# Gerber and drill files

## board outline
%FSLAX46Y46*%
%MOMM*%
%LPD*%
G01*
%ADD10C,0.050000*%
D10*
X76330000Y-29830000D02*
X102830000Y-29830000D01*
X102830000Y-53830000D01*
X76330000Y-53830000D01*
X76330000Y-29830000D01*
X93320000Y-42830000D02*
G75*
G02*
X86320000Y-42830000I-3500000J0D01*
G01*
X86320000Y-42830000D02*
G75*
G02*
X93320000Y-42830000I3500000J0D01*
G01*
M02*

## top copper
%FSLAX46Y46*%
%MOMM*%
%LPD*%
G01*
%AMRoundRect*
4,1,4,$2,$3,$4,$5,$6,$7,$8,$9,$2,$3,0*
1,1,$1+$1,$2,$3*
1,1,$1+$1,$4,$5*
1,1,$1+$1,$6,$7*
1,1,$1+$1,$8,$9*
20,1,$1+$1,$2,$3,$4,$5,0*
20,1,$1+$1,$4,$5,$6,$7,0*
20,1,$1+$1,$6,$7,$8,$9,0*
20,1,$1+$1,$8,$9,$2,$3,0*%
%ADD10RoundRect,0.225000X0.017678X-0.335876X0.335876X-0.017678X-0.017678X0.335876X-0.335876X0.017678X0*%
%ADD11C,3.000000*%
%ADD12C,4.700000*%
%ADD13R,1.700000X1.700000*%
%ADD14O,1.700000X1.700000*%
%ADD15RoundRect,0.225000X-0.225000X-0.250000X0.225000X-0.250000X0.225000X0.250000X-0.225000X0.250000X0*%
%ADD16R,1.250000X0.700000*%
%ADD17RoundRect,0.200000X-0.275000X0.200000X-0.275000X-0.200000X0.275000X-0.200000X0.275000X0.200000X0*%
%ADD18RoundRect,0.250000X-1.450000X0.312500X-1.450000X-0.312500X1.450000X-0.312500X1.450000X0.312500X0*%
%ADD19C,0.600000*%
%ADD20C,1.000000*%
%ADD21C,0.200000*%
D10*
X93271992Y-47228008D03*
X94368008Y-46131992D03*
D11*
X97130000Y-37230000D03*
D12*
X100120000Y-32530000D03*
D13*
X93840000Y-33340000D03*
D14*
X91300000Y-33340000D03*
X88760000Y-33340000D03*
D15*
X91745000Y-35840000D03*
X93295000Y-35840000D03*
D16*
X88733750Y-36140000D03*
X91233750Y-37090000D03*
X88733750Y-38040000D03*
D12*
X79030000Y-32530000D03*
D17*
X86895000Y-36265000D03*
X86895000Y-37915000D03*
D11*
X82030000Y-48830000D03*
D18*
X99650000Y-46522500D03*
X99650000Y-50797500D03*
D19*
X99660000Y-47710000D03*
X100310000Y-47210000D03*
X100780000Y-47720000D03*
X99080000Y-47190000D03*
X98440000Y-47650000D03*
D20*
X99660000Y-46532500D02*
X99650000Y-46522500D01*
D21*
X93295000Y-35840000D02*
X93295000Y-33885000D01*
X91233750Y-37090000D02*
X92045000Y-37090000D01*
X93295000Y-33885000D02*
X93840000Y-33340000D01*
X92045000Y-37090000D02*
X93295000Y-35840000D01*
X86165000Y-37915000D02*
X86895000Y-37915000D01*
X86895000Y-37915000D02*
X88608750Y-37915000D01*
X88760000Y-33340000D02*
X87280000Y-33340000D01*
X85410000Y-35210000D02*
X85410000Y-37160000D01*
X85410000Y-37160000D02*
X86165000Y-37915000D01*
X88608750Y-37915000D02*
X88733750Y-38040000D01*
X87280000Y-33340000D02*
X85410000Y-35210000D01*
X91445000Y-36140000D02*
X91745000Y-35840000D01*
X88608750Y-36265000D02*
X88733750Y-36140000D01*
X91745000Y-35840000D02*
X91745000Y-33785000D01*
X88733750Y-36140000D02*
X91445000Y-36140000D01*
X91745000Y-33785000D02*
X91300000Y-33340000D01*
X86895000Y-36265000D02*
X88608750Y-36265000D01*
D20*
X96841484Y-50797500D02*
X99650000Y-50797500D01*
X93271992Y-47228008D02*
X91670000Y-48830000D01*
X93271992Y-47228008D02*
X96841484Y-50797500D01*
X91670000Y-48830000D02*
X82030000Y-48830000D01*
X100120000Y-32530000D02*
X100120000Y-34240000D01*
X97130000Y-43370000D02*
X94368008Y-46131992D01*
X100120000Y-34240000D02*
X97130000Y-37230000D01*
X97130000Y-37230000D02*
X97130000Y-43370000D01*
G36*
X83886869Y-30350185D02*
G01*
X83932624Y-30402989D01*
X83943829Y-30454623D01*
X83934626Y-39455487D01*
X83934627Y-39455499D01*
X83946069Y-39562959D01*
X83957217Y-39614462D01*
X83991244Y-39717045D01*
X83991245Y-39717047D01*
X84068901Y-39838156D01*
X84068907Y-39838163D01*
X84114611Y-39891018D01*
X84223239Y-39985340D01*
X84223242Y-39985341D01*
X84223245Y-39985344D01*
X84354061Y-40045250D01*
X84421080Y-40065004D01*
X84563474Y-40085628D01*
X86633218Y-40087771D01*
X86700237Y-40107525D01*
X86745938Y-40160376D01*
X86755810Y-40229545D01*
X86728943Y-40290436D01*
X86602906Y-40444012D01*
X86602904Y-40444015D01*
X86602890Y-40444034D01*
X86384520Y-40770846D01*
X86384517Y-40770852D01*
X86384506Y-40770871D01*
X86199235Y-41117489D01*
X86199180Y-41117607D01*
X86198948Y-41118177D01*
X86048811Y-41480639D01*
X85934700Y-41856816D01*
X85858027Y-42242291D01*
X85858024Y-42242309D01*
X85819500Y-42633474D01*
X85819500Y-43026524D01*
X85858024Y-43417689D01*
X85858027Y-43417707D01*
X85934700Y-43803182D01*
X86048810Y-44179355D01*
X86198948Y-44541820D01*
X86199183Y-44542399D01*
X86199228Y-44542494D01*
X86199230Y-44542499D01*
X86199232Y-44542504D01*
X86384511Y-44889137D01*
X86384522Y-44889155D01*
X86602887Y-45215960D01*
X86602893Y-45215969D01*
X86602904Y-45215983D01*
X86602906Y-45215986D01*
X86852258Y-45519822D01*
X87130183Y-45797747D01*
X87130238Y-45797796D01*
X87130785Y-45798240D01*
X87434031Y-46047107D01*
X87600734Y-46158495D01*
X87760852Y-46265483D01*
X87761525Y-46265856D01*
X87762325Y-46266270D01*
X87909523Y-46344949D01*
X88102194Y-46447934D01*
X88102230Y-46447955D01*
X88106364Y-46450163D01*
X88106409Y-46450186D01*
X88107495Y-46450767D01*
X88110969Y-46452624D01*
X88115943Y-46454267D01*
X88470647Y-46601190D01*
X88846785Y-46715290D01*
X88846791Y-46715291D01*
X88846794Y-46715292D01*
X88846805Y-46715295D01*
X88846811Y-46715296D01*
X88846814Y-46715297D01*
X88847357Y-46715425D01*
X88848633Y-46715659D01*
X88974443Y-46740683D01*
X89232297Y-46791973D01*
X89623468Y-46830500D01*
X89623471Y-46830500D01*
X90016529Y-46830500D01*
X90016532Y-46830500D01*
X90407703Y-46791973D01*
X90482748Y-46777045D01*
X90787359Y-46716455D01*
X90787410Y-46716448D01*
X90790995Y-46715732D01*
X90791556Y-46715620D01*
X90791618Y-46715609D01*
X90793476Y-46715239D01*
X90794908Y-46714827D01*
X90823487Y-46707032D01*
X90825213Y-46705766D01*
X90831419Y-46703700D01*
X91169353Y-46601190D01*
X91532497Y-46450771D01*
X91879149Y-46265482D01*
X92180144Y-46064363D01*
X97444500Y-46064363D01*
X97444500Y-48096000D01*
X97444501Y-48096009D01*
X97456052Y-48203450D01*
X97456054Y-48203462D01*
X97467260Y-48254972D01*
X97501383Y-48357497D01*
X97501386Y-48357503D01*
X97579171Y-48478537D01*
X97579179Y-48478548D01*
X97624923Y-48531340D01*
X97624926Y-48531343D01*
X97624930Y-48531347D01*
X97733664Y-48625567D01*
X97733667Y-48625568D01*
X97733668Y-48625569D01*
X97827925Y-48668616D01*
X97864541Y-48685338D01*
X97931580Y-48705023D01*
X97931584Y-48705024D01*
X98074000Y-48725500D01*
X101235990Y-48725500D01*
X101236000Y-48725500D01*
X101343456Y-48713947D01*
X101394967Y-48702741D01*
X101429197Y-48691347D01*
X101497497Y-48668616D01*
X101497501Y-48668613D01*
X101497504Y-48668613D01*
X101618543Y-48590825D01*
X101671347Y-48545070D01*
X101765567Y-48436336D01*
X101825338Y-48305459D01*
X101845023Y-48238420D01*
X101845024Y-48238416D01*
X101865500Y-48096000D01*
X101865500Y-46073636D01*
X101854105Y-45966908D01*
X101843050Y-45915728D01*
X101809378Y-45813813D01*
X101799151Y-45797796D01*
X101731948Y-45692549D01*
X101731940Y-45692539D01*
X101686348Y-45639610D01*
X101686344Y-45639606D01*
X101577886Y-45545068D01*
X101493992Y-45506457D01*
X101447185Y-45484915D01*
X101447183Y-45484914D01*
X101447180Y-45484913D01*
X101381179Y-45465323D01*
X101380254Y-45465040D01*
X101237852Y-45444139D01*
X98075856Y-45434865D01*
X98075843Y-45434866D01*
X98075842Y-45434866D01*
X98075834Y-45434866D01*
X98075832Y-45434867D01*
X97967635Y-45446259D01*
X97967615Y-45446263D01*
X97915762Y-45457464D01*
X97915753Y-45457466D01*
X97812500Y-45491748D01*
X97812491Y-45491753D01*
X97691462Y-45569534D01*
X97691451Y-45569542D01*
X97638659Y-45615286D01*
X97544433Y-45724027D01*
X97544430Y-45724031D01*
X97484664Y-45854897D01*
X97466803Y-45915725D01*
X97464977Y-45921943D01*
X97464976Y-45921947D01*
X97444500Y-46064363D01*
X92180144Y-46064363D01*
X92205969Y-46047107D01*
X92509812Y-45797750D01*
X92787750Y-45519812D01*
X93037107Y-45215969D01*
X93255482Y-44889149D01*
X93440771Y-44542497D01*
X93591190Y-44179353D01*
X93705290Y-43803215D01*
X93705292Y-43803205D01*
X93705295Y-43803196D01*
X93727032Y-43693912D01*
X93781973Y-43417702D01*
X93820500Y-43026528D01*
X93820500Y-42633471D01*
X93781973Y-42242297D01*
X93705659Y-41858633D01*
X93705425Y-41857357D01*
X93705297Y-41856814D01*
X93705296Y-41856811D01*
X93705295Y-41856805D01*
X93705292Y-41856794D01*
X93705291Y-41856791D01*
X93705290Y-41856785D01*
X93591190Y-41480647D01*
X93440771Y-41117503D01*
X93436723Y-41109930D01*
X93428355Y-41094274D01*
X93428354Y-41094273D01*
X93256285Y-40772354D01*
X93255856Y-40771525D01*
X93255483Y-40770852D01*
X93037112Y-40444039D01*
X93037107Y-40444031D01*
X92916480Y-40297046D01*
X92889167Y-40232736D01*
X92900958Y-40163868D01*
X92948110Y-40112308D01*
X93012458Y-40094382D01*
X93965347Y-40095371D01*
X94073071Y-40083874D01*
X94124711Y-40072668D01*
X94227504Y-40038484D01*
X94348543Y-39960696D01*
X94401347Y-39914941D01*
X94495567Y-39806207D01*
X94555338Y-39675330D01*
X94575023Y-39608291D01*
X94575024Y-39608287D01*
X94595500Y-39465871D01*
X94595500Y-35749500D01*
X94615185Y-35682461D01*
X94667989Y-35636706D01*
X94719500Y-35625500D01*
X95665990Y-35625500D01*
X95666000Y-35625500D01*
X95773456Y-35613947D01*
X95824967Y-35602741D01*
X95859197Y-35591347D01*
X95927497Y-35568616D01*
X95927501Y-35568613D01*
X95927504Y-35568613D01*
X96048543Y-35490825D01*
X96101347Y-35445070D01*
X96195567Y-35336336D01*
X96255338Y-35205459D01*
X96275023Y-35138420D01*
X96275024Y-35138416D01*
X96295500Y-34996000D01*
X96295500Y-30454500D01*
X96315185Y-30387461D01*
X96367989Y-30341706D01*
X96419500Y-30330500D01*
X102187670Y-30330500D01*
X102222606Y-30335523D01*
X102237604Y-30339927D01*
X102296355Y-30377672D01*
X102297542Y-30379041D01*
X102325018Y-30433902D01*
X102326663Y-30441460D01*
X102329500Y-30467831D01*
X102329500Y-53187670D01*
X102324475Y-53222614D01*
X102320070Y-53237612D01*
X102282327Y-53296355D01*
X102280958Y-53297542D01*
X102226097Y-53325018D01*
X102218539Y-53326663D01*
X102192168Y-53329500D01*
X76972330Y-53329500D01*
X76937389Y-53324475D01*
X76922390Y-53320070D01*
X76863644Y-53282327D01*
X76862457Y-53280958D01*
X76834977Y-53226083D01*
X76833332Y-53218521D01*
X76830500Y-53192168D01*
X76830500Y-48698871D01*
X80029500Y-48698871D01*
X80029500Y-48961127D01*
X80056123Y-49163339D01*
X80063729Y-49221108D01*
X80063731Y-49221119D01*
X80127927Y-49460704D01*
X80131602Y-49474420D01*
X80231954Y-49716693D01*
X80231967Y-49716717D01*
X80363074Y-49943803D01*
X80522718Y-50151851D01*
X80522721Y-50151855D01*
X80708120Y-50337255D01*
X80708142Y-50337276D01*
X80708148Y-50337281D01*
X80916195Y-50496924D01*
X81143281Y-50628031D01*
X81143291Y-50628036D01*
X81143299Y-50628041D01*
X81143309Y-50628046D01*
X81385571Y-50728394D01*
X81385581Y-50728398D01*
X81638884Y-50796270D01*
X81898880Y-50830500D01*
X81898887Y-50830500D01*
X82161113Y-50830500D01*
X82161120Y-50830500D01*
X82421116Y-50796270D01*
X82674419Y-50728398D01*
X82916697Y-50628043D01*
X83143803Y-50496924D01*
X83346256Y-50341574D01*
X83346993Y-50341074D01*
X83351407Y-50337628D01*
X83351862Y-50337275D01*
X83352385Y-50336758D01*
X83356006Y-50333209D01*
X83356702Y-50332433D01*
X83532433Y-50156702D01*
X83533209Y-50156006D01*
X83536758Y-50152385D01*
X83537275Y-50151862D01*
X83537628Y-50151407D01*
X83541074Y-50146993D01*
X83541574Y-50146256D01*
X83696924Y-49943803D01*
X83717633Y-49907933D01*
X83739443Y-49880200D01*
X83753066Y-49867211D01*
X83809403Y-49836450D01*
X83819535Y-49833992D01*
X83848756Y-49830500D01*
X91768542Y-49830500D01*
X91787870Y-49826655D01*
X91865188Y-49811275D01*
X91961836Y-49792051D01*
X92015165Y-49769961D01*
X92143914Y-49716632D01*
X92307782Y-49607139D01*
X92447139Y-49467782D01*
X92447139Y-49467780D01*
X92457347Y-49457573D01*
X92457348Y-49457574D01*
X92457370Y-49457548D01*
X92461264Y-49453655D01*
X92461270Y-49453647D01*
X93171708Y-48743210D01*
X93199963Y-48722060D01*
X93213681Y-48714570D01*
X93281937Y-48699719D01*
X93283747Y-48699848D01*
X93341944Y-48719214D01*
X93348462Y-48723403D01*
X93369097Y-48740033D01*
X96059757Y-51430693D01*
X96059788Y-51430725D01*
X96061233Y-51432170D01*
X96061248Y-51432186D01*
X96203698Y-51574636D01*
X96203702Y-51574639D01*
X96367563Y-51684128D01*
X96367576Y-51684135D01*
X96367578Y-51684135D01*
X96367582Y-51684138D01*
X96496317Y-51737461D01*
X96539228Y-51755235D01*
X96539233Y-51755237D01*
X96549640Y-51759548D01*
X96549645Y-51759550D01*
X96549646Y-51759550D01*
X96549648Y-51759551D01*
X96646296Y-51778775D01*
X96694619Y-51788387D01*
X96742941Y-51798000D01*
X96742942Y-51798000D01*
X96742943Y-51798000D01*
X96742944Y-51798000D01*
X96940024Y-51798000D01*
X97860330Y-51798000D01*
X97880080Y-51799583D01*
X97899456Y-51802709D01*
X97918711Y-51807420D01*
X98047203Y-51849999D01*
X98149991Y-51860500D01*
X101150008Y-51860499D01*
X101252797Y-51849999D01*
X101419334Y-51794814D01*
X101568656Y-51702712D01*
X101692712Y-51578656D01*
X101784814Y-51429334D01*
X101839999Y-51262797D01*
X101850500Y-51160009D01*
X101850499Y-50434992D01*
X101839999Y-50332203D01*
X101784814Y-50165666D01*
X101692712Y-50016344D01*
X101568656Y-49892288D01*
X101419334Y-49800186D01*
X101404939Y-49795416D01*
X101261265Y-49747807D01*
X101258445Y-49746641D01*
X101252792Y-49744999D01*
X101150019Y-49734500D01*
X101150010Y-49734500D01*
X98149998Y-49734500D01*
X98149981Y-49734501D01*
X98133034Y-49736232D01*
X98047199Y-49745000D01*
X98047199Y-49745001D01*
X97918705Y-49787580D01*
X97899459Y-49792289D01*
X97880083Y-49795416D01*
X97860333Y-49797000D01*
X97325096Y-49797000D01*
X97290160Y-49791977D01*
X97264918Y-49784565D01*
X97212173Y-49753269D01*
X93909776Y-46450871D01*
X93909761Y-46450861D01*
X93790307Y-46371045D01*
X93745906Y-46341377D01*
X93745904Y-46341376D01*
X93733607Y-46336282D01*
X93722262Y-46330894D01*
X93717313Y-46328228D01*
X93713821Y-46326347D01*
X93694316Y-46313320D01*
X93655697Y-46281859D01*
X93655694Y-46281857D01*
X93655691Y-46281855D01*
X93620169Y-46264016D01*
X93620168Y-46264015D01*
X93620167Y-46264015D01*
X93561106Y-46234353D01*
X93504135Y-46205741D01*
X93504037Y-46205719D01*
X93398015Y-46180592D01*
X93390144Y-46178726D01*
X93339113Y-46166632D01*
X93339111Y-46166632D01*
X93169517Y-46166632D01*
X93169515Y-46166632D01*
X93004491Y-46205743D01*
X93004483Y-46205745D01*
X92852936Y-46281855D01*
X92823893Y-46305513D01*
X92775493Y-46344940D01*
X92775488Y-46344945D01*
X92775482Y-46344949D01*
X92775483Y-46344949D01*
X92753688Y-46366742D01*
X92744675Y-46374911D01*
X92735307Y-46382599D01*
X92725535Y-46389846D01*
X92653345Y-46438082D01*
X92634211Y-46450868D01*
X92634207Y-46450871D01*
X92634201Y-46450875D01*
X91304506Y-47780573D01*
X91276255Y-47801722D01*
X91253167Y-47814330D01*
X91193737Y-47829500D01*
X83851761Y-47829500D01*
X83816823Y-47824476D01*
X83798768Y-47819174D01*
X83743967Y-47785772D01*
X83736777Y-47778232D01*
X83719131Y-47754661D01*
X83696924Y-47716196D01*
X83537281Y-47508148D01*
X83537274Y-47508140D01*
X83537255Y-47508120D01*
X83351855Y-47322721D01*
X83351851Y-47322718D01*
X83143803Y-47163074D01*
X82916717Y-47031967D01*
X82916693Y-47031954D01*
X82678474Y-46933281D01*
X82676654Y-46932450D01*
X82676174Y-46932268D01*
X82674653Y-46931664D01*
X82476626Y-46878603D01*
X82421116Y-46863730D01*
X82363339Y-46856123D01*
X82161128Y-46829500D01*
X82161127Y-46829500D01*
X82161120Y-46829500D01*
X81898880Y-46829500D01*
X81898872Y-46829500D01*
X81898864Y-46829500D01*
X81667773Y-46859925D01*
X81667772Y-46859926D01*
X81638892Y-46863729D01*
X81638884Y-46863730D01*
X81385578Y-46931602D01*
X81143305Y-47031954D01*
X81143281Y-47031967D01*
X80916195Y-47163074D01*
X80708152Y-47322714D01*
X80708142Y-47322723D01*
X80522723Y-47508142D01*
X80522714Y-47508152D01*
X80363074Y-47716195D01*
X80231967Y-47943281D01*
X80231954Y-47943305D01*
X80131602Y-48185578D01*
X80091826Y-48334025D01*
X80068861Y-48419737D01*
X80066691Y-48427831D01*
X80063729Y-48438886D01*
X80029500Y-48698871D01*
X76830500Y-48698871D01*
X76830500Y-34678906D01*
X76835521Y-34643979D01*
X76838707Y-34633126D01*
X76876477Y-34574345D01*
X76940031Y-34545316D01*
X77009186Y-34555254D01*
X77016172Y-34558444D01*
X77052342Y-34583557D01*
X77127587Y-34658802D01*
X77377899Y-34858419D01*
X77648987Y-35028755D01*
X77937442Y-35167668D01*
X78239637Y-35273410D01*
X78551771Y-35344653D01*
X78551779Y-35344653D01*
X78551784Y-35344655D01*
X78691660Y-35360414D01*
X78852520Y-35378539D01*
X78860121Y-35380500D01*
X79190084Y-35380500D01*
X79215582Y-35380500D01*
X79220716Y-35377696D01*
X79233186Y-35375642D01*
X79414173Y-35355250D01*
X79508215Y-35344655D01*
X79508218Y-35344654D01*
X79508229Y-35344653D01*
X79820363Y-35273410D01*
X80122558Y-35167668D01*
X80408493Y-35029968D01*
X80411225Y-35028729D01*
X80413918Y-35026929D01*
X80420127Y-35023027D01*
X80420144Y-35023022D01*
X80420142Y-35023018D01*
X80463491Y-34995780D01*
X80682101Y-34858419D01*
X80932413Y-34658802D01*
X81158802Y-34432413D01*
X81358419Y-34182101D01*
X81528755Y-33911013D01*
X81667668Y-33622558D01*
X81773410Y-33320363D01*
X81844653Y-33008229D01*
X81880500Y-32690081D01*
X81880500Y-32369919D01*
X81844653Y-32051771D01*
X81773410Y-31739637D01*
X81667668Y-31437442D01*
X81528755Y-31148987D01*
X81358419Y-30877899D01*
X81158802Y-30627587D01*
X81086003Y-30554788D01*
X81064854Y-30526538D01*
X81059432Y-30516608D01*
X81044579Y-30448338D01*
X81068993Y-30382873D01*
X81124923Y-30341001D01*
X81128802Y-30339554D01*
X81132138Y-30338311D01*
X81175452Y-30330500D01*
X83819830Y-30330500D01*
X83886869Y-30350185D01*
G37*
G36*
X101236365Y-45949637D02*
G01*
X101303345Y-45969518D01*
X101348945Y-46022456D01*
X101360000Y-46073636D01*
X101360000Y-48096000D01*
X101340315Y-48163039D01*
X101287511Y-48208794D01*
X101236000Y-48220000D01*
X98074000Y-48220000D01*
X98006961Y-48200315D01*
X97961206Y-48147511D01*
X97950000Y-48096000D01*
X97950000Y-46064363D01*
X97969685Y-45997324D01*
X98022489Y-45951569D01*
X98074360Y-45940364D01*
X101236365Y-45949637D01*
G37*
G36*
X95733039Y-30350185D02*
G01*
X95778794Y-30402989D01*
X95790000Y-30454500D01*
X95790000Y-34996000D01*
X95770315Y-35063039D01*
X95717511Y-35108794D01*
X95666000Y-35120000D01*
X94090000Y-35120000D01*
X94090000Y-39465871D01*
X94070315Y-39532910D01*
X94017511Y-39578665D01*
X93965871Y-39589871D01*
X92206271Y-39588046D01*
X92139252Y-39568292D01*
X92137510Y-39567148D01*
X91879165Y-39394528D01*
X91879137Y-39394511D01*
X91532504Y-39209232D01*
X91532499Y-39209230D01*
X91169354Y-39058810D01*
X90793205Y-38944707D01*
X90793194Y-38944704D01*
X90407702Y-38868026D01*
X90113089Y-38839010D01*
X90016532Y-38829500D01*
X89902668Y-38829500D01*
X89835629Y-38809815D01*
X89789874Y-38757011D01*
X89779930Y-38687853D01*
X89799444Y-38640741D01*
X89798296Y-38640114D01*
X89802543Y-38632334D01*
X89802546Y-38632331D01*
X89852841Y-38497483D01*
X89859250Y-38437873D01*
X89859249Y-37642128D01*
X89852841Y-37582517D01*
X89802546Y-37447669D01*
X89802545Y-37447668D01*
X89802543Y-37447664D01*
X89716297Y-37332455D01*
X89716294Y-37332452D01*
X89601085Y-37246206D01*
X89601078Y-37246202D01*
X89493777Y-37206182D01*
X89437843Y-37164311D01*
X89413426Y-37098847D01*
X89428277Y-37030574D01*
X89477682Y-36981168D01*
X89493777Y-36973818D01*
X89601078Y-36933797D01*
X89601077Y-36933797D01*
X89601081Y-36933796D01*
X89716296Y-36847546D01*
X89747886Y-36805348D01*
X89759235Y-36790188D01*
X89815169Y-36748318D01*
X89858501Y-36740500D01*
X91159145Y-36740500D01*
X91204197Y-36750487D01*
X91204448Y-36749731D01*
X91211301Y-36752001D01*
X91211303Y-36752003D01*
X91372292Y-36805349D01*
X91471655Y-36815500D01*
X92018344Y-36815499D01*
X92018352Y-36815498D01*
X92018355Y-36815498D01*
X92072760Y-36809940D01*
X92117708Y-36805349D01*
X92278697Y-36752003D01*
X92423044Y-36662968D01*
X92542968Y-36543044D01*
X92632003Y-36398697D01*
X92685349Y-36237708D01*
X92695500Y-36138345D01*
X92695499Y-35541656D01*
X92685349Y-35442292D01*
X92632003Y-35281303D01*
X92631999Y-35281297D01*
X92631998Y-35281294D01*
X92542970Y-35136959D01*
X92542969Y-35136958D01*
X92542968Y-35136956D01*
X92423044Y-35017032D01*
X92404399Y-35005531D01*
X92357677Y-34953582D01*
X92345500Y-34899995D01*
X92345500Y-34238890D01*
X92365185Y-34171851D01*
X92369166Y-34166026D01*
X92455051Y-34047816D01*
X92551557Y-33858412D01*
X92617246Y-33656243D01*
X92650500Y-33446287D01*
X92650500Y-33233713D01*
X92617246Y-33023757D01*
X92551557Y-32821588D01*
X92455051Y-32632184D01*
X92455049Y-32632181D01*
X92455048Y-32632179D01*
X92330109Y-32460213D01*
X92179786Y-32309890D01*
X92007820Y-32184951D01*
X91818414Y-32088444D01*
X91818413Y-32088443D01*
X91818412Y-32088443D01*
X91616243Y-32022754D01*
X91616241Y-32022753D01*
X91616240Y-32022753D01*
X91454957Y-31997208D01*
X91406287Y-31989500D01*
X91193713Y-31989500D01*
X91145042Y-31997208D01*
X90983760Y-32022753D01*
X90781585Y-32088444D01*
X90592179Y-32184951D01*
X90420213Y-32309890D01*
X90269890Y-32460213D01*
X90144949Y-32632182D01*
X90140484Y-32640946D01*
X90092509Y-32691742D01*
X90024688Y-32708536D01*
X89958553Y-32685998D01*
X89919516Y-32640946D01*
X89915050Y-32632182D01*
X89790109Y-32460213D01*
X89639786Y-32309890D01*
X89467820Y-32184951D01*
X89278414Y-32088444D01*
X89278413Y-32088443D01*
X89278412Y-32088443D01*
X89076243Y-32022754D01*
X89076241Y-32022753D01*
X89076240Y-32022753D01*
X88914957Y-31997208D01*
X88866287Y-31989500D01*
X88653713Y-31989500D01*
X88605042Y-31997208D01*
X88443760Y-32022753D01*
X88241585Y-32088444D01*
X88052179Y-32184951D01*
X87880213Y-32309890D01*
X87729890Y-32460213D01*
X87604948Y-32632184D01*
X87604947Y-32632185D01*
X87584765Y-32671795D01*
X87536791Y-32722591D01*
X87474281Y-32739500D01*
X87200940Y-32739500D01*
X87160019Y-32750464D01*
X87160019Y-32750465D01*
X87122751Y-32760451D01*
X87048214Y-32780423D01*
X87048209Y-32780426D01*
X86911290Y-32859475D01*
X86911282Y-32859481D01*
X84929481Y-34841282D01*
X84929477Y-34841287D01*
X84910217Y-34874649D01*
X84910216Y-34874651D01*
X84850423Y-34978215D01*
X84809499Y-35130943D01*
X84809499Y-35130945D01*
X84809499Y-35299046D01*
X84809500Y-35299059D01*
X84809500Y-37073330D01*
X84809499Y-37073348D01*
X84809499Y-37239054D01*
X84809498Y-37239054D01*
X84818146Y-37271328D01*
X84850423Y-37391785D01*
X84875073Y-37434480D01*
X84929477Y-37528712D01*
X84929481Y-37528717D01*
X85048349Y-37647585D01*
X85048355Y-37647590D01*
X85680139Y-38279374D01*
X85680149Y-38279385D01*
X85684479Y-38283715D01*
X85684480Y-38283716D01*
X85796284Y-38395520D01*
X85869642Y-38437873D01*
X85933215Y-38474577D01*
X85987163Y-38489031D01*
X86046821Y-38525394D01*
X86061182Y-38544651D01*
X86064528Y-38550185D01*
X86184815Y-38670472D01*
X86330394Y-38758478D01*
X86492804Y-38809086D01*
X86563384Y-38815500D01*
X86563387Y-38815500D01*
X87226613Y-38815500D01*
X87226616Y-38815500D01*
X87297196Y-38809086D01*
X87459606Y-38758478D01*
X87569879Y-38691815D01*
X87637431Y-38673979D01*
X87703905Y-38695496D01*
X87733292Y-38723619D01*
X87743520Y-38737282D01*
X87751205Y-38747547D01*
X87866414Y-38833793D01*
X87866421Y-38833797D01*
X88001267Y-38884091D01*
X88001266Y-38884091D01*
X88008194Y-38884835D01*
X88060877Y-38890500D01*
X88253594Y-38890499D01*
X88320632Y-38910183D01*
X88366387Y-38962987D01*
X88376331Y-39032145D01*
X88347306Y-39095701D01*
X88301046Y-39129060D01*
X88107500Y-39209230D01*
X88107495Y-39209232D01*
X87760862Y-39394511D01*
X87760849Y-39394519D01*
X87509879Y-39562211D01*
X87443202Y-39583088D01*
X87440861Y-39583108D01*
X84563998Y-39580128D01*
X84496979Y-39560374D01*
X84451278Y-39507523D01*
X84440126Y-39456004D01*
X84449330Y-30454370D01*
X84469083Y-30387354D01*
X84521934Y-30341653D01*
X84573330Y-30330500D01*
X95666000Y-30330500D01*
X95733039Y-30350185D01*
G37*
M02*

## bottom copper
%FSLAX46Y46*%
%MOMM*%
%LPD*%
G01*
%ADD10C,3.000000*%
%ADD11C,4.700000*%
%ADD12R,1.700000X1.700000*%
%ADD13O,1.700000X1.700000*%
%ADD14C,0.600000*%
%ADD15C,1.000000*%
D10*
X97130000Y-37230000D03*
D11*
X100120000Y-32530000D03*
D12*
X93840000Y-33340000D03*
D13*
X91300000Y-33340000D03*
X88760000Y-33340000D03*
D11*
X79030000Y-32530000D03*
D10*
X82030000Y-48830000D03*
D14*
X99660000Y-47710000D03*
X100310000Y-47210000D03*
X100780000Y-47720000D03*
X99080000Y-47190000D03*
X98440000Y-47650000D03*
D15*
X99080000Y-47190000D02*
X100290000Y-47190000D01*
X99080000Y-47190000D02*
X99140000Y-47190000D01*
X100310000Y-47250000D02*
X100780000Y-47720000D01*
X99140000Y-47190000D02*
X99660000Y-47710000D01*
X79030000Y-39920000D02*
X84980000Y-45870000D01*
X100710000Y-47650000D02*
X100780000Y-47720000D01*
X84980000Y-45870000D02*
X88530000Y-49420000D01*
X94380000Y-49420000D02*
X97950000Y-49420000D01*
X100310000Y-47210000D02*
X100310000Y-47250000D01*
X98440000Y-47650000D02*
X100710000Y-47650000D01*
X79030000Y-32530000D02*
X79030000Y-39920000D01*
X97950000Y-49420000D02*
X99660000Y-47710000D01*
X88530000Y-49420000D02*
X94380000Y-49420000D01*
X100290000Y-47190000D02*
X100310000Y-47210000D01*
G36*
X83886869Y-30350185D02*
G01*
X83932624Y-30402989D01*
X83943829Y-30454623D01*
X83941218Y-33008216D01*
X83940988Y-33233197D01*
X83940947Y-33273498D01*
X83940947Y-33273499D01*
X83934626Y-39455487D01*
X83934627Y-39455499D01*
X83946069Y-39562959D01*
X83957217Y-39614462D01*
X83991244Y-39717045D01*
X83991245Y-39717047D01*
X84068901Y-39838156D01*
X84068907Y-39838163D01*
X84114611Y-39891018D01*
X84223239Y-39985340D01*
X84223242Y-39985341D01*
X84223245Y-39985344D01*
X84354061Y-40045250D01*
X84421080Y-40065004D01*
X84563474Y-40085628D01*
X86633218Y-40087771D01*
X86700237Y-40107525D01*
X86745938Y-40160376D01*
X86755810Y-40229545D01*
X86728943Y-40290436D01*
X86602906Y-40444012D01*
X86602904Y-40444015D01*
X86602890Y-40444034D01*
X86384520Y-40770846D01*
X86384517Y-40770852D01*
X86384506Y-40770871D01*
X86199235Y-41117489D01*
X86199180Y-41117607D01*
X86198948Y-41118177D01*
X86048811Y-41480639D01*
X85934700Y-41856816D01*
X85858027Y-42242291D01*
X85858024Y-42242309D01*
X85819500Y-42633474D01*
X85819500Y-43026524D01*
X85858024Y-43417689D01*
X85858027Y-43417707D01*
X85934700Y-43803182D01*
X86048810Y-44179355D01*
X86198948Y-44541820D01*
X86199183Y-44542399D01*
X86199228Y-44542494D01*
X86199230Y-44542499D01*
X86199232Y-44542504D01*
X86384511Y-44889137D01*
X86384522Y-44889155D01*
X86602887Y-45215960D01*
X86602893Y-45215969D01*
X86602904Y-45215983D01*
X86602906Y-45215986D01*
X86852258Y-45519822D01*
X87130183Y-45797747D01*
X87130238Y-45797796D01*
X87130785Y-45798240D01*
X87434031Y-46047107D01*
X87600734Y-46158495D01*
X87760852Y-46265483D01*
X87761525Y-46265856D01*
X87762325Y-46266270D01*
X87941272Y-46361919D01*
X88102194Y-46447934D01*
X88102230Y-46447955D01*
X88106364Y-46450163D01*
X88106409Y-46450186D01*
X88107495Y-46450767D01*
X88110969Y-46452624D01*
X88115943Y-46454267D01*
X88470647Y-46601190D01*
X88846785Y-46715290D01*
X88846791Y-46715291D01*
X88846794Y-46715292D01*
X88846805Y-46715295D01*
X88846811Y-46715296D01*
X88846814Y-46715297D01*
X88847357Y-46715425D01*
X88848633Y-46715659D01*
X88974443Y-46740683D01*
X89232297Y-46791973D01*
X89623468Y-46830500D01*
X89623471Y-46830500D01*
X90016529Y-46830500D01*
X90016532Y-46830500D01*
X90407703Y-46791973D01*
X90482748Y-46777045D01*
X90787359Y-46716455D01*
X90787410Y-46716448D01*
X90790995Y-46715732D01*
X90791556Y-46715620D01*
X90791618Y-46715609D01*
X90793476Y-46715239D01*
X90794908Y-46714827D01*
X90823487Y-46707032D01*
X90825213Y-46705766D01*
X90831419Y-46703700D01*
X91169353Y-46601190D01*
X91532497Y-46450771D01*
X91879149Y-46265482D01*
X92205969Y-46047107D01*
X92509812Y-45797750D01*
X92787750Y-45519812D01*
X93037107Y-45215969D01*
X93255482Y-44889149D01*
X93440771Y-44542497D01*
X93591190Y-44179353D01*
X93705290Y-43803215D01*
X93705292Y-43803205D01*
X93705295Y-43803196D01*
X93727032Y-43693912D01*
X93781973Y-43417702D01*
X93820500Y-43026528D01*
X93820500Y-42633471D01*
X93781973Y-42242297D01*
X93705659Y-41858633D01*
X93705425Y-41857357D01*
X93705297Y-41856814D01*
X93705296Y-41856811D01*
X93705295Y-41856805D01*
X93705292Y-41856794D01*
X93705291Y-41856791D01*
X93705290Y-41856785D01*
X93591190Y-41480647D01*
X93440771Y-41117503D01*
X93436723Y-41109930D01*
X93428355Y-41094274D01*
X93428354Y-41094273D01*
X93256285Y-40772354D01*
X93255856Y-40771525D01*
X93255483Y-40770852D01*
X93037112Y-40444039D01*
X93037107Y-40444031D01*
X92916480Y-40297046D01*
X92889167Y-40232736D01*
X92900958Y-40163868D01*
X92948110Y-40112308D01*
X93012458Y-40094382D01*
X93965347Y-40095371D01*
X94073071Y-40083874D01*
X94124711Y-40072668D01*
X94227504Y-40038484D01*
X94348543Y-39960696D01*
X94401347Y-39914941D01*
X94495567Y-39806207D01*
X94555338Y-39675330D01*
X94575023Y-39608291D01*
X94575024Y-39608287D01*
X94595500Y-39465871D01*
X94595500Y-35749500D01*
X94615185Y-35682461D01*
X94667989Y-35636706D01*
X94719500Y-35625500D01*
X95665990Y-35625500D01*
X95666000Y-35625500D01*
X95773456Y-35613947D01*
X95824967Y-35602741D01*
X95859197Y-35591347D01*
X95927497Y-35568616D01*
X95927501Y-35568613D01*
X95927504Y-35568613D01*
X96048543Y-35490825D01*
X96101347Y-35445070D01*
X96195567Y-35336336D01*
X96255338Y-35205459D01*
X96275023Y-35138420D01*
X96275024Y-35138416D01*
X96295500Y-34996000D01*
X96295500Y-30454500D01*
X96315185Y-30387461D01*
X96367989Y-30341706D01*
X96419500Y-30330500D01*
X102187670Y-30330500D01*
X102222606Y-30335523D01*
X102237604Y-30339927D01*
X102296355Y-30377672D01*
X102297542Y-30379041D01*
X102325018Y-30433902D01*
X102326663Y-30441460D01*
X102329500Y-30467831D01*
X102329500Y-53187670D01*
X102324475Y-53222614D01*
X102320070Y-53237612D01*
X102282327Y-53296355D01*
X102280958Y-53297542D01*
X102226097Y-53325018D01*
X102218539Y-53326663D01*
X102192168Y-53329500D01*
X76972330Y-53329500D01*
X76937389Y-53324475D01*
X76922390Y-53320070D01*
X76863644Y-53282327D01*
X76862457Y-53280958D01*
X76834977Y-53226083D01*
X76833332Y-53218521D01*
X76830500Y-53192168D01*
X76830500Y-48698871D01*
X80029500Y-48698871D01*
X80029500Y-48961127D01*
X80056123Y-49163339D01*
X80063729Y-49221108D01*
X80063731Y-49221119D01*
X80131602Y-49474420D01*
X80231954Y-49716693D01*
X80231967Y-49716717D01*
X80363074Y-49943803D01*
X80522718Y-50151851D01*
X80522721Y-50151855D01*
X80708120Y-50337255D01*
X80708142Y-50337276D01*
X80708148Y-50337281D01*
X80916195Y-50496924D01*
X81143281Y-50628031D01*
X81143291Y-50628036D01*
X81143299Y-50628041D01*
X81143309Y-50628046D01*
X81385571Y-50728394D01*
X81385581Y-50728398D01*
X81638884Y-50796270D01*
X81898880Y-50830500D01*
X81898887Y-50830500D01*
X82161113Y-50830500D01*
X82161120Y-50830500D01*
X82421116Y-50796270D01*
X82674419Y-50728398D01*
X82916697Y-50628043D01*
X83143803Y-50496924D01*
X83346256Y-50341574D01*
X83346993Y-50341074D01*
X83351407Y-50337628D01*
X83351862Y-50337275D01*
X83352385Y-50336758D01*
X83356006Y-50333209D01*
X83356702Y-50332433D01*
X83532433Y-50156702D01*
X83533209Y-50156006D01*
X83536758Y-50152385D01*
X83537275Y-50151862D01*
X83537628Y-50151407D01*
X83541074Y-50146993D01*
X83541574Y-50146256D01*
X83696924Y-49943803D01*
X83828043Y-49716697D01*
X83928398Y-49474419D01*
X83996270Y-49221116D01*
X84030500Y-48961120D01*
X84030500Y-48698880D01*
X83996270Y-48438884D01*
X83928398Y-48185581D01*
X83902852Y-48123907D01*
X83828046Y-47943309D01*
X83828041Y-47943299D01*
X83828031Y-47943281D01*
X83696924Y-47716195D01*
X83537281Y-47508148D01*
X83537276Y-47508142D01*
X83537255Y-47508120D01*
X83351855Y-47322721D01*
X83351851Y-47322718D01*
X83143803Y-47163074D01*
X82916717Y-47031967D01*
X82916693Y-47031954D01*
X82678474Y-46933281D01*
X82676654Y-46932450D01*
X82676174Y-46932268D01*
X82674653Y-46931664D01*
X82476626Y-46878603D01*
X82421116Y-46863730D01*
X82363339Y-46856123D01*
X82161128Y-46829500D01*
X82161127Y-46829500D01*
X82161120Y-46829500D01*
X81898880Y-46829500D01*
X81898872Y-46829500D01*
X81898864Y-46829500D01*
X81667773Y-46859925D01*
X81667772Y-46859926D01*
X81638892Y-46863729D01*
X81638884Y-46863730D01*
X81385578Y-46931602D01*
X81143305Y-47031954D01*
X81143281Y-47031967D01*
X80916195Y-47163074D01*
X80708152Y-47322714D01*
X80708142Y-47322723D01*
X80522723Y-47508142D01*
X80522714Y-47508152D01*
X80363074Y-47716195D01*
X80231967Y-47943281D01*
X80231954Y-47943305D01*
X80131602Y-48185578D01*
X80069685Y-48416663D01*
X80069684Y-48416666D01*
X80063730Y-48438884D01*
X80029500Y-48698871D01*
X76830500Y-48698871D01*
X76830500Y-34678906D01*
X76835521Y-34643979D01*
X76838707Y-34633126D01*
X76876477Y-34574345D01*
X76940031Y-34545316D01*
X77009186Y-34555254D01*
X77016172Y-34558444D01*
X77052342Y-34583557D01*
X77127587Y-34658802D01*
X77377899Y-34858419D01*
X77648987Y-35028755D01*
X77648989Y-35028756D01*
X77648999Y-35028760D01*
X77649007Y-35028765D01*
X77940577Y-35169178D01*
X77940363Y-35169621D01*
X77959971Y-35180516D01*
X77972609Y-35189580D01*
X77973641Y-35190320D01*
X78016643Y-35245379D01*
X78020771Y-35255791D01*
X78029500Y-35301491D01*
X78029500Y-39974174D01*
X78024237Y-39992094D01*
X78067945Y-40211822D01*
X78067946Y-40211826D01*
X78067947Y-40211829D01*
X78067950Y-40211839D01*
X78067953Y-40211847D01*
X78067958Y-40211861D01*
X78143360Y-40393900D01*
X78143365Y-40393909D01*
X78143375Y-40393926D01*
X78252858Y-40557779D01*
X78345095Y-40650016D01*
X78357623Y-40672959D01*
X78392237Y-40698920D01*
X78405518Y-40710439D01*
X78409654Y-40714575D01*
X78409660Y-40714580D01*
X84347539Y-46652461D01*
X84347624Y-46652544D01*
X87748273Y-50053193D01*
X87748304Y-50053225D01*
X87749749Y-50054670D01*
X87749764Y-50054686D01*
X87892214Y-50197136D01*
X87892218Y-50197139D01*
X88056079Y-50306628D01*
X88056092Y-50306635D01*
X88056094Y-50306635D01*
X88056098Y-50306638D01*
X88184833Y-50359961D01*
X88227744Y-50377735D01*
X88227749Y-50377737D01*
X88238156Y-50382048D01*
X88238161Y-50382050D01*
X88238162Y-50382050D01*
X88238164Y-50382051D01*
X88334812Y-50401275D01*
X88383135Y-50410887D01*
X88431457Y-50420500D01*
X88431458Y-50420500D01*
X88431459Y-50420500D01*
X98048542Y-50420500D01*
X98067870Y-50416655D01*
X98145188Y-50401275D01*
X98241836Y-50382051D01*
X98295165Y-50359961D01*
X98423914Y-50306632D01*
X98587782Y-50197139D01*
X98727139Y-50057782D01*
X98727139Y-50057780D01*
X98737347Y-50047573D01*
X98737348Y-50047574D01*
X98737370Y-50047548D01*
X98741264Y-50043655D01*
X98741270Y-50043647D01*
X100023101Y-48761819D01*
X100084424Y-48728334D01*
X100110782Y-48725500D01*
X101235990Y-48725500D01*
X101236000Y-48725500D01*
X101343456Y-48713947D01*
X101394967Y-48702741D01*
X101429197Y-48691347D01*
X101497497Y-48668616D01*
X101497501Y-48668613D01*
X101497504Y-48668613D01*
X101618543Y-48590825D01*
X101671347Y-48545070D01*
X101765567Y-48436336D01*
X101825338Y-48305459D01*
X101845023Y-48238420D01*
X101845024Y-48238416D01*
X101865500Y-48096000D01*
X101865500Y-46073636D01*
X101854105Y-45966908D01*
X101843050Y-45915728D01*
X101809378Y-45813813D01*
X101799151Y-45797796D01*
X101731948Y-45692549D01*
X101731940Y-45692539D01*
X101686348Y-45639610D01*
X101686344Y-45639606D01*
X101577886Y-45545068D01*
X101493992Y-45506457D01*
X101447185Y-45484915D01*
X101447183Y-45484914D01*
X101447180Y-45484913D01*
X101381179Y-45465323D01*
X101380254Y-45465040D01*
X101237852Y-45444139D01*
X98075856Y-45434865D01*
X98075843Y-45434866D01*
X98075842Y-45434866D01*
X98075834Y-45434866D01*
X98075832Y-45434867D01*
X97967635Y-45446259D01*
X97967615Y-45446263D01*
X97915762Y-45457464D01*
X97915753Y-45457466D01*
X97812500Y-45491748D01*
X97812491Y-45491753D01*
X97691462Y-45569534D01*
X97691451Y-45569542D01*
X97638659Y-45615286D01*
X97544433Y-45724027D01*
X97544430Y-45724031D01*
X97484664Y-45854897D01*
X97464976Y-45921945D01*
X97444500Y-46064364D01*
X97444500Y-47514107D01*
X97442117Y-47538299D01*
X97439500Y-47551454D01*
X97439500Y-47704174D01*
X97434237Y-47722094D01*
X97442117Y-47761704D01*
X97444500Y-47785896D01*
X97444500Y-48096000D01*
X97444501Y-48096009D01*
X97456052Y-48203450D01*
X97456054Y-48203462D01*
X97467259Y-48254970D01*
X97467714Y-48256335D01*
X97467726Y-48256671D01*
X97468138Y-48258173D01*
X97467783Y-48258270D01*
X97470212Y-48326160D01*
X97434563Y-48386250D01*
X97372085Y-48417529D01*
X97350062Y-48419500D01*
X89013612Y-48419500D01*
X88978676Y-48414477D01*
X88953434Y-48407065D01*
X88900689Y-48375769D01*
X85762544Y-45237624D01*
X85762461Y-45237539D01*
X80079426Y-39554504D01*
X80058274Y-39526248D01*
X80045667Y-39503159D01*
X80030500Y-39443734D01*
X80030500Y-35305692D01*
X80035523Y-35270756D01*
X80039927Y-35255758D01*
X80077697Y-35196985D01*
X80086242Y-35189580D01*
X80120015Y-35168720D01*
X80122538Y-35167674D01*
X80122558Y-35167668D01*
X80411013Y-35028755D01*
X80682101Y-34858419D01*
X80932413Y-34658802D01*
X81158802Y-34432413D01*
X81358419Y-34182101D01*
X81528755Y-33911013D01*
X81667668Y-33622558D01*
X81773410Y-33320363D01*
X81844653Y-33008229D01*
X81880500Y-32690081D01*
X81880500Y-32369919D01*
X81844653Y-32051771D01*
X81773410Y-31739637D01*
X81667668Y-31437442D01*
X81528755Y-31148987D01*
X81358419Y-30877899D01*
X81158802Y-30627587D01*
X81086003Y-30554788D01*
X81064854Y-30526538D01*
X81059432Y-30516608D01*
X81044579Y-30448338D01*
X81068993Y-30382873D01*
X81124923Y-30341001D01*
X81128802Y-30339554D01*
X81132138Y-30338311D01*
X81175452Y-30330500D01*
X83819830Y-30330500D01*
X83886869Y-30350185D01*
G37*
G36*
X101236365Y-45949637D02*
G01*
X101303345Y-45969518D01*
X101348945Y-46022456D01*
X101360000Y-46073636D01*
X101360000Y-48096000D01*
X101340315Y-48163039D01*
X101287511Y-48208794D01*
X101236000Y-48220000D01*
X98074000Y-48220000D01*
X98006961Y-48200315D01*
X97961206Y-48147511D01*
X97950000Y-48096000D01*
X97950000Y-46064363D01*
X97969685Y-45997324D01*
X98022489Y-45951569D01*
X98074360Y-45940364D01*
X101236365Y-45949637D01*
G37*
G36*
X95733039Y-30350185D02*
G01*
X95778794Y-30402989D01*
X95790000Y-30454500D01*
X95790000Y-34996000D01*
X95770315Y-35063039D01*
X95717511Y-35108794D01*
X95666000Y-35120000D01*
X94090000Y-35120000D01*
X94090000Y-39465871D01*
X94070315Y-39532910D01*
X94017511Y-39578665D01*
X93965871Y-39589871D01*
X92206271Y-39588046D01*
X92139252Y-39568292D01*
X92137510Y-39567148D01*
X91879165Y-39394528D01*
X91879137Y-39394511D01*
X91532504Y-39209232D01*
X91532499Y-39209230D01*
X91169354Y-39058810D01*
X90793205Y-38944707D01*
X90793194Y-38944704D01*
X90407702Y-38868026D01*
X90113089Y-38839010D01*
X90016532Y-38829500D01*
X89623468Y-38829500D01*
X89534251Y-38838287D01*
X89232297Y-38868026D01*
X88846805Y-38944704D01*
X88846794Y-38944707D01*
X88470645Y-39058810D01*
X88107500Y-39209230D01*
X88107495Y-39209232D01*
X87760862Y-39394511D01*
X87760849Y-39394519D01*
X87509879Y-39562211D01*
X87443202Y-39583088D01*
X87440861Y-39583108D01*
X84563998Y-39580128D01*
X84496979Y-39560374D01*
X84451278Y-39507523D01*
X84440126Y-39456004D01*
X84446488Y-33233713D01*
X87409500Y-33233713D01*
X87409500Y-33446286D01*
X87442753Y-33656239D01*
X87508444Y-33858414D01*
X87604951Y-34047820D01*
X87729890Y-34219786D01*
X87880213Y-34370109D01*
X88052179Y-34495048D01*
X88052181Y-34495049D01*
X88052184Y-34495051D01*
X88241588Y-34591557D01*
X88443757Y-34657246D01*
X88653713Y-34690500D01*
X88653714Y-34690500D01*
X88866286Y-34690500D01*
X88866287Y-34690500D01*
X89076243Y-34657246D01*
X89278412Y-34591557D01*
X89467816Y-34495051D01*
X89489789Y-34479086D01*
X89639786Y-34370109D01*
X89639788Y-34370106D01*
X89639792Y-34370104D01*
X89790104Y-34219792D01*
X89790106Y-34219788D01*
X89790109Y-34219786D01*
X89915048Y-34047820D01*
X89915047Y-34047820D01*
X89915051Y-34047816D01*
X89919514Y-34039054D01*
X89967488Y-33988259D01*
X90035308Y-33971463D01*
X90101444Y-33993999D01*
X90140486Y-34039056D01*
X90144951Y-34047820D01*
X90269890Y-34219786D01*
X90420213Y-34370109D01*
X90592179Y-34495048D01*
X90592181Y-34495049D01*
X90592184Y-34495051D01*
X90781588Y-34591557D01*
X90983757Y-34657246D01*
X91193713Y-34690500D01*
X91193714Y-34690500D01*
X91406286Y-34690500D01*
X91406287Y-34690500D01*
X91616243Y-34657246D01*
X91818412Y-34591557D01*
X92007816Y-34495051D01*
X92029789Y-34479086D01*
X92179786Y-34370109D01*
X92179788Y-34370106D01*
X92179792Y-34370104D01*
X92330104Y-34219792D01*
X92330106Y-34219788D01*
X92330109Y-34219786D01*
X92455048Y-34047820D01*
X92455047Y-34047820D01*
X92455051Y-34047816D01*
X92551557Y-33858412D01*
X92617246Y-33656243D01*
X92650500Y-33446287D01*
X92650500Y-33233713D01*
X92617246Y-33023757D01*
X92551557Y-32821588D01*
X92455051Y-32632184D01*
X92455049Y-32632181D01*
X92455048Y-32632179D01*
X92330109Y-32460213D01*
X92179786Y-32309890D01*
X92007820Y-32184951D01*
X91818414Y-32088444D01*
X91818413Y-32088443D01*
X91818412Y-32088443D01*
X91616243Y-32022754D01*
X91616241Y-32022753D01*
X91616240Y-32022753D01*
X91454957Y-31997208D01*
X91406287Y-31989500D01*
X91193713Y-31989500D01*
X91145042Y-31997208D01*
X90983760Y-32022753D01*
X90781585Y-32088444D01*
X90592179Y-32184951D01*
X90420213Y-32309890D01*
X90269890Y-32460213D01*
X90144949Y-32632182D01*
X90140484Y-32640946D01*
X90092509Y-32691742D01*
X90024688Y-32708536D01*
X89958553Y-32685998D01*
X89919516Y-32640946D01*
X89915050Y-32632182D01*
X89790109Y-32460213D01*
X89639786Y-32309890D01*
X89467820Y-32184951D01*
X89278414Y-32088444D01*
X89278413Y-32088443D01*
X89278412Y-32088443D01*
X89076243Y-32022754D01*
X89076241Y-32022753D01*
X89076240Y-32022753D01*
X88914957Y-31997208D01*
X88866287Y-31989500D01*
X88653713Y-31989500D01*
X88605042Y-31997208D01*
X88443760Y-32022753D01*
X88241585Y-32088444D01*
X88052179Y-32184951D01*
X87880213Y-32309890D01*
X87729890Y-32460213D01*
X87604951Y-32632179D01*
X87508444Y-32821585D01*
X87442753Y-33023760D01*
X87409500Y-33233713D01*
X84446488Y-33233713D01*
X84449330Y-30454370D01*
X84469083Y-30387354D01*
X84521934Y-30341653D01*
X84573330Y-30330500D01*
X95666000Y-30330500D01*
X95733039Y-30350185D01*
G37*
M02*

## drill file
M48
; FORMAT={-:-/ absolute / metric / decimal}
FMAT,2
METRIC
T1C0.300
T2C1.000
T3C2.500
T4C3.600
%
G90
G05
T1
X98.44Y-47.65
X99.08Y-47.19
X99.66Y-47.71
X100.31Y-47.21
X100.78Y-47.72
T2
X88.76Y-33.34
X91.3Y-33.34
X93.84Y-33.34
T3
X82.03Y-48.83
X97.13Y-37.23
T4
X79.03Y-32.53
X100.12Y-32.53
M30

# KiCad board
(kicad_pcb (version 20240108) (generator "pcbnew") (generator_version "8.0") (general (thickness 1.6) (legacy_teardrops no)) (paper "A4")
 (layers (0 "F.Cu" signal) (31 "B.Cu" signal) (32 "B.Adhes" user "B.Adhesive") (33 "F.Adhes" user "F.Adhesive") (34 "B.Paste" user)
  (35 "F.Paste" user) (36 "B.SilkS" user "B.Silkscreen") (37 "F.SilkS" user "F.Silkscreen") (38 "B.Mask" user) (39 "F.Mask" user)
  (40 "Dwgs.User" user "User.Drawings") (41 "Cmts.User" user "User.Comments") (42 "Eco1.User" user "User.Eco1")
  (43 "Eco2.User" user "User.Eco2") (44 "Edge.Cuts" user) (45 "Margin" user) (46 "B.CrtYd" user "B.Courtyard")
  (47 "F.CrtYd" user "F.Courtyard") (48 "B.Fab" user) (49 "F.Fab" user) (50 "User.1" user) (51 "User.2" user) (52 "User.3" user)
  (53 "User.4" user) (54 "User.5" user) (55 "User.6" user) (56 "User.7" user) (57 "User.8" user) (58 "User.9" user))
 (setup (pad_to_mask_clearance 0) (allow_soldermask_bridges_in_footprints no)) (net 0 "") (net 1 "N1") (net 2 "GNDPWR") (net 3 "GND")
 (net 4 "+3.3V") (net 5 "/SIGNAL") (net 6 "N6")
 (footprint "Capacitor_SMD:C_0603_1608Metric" (layer "F.Cu") (at 93.82 46.68 45)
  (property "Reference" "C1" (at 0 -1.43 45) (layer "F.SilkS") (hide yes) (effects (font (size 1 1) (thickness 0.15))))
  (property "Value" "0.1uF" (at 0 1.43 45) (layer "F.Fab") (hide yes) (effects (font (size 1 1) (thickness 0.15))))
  (pad "1" smd roundrect (at -0.775 0 45) (size 0.9 0.95) (layers "F.Cu" "F.Paste" "F.Mask") (roundrect_rratio 0.25) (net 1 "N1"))
  (pad "2" smd roundrect (at 0.775 0 45) (size 0.9 0.95) (layers "F.Cu" "F.Paste" "F.Mask") (roundrect_rratio 0.25) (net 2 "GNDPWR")))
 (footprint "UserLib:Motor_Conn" (layer "F.Cu") (at 97.13 37.23)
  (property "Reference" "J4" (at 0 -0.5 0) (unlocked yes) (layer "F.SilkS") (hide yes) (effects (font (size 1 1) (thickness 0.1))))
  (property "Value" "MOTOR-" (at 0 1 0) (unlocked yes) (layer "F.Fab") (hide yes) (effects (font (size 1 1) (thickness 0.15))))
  (pad "1" thru_hole circle (at 0 0) (size 3 3) (drill 2.5) (layers "*.Cu" "*.Mask") (remove_unused_layers no) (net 2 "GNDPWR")))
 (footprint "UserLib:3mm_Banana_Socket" (layer "F.Cu") (at 100.12 32.53)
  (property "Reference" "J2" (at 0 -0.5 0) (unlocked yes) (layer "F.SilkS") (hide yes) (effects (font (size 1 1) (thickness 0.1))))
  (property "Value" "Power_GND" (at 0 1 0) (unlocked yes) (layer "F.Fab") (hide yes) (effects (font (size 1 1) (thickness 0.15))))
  (pad "1" thru_hole circle (at 0 0) (size 4.7 4.7) (drill 3.6) (layers "*.Cu" "*.Mask") (remove_unused_layers no) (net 2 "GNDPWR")))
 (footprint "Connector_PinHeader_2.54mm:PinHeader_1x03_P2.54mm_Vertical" (layer "F.Cu") (at 93.84 33.34 -90)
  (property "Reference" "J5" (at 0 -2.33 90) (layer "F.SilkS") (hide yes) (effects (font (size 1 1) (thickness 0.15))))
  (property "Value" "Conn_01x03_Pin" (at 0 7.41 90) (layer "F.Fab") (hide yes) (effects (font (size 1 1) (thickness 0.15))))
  (pad "1" thru_hole rect (at 0 0 270) (size 1.7 1.7) (drill 1) (layers "*.Cu" "*.Mask") (remove_unused_layers no) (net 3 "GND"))
  (pad "2" thru_hole oval (at 0 2.54 270) (size 1.7 1.7) (drill 1) (layers "*.Cu" "*.Mask") (remove_unused_layers no) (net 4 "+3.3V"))
  (pad "3" thru_hole oval (at 0 5.08 270) (size 1.7 1.7) (drill 1) (layers "*.Cu" "*.Mask") (remove_unused_layers no) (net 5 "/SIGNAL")))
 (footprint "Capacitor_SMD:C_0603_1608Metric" (layer "F.Cu") (at 92.52 35.84)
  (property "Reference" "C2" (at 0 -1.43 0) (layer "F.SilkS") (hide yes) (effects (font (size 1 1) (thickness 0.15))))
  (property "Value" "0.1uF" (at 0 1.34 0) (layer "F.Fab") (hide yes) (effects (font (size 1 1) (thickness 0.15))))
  (pad "1" smd roundrect (at -0.775 0) (size 0.9 0.95) (layers "F.Cu" "F.Paste" "F.Mask") (roundrect_rratio 0.25) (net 4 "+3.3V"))
  (pad "2" smd roundrect (at 0.775 0) (size 0.9 0.95) (layers "F.Cu" "F.Paste" "F.Mask") (roundrect_rratio 0.25) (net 3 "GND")))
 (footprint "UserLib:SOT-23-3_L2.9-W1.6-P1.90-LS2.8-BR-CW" (layer "F.Cu") (at 89.98375 37.09 180)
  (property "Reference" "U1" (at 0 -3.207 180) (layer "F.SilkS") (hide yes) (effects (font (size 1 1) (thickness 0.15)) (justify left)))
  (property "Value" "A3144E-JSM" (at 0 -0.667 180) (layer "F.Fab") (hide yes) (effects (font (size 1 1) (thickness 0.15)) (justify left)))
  (pad "1" smd rect (at 1.25 0.95 90) (size 0.7 1.25) (layers "F.Cu" "F.Paste" "F.Mask") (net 4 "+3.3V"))
  (pad "2" smd rect (at -1.25 0 90) (size 0.7 1.25) (layers "F.Cu" "F.Paste" "F.Mask") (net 3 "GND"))
  (pad "3" smd rect (at 1.25 -0.95 90) (size 0.7 1.25) (layers "F.Cu" "F.Paste" "F.Mask") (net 5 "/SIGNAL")))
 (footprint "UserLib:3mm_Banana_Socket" (layer "F.Cu") (at 79.03 32.53)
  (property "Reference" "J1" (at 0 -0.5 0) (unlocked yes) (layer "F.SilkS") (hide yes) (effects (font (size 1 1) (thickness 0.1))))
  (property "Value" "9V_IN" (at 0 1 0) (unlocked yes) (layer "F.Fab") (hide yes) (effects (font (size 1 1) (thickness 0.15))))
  (pad "1" thru_hole circle (at 0 0) (size 4.7 4.7) (drill 3.6) (layers "*.Cu" "*.Mask") (remove_unused_layers no) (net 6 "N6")))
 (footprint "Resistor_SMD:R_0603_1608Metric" (layer "F.Cu") (at 86.895 37.09 -90)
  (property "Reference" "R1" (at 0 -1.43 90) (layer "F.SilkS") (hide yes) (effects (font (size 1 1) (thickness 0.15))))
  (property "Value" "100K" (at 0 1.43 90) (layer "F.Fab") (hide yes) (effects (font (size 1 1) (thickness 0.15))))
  (pad "1" smd roundrect (at -0.825 0 270) (size 0.8 0.95) (layers "F.Cu" "F.Paste" "F.Mask") (roundrect_rratio 0.25) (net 4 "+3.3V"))
  (pad "2" smd roundrect (at 0.825 0 270) (size 0.8 0.95) (layers "F.Cu" "F.Paste" "F.Mask") (roundrect_rratio 0.25) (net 5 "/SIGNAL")))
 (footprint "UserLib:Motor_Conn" (layer "F.Cu") (at 82.03 48.83)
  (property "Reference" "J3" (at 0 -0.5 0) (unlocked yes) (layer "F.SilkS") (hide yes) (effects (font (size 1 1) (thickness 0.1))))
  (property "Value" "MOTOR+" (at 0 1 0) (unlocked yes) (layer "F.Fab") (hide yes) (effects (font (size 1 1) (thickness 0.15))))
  (pad "1" thru_hole circle (at 0 0) (size 3 3) (drill 2.5) (layers "*.Cu" "*.Mask") (remove_unused_layers no) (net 1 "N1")))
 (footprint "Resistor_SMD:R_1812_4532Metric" (layer "F.Cu") (at 99.65 48.66 -90)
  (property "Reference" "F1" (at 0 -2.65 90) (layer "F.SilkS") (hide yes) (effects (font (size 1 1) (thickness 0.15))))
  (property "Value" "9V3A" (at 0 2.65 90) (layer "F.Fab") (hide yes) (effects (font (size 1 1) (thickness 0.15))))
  (pad "1" smd roundrect (at -2.1375 0 270) (size 1.125 3.4) (layers "F.Cu" "F.Paste" "F.Mask") (roundrect_rratio 0.222222) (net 6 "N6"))
  (pad "2" smd roundrect (at 2.1375 0 270) (size 1.125 3.4) (layers "F.Cu" "F.Paste" "F.Mask") (roundrect_rratio 0.222222) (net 1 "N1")))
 (gr_rect (start 76.33 29.83) (end 102.83 53.83) (stroke (width 0.05) (type default)) (fill none) (layer "Edge.Cuts"))
 (gr_circle (center 89.82 42.83) (end 93.32 42.83) (stroke (width 0.05) (type default)) (fill none) (layer "Edge.Cuts"))
 (segment (start 99.66 46.5325) (end 99.65 46.5225) (width 1) (layer "F.Cu") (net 6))
 (via (at 99.66 47.71) (size 0.6) (drill 0.3) (layers "F.Cu" "B.Cu") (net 6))
 (via (at 100.31 47.21) (size 0.6) (drill 0.3) (layers "F.Cu" "B.Cu") (free yes) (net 6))
 (via (at 100.78 47.72) (size 0.6) (drill 0.3) (layers "F.Cu" "B.Cu") (free yes) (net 6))
 (via (at 99.08 47.19) (size 0.6) (drill 0.3) (layers "F.Cu" "B.Cu") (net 6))
 (via (at 98.44 47.65) (size 0.6) (drill 0.3) (layers "F.Cu" "B.Cu") (free yes) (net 6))
 (segment (start 99.08 47.19) (end 100.29 47.19) (width 1) (layer "B.Cu") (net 6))
 (segment (start 99.08 47.19) (end 99.14 47.19) (width 1) (layer "B.Cu") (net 6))
 (segment (start 100.31 47.25) (end 100.78 47.72) (width 1) (layer "B.Cu") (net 6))
 (segment (start 99.14 47.19) (end 99.66 47.71) (width 1) (layer "B.Cu") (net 6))
 (segment (start 79.03 39.92) (end 84.98 45.87) (width 1) (layer "B.Cu") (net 6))
 (segment (start 100.71 47.65) (end 100.78 47.72) (width 1) (layer "B.Cu") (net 6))
 (segment (start 84.98 45.87) (end 88.53 49.42) (width 1) (layer "B.Cu") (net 6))
 (segment (start 94.38 49.42) (end 97.95 49.42) (width 1) (layer "B.Cu") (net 6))
 (segment (start 100.31 47.21) (end 100.31 47.25) (width 1) (layer "B.Cu") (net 6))
 (segment (start 98.44 47.65) (end 100.71 47.65) (width 1) (layer "B.Cu") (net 6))
 (segment (start 79.03 32.53) (end 79.03 39.92) (width 1) (layer "B.Cu") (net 6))
 (segment (start 97.95 49.42) (end 99.66 47.71) (width 1) (layer "B.Cu") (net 6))
 (segment (start 88.53 49.42) (end 94.38 49.42) (width 1) (layer "B.Cu") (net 6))
 (segment (start 100.29 47.19) (end 100.31 47.21) (width 1) (layer "B.Cu") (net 6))
 (segment (start 93.295 35.84) (end 93.295 33.885) (width 0.2) (layer "F.Cu") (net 3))
 (segment (start 91.23375 37.09) (end 92.045 37.09) (width 0.2) (layer "F.Cu") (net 3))
 (segment (start 93.295 33.885) (end 93.84 33.34) (width 0.2) (layer "F.Cu") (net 3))
 (segment (start 92.045 37.09) (end 93.295 35.84) (width 0.2) (layer "F.Cu") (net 3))
 (segment (start 86.165 37.915) (end 86.895 37.915) (width 0.2) (layer "F.Cu") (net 5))
 (segment (start 86.895 37.915) (end 88.60875 37.915) (width 0.2) (layer "F.Cu") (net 5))
 (segment (start 88.76 33.34) (end 87.28 33.34) (width 0.2) (layer "F.Cu") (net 5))
 (segment (start 85.41 35.21) (end 85.41 37.16) (width 0.2) (layer "F.Cu") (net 5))
 (segment (start 85.41 37.16) (end 86.165 37.915) (width 0.2) (layer "F.Cu") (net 5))
 (segment (start 88.60875 37.915) (end 88.73375 38.04) (width 0.2) (layer "F.Cu") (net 5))
 (segment (start 87.28 33.34) (end 85.41 35.21) (width 0.2) (layer "F.Cu") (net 5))
 (segment (start 91.445 36.14) (end 91.745 35.84) (width 0.2) (layer "F.Cu") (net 4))
 (segment (start 88.60875 36.265) (end 88.73375 36.14) (width 0.2) (layer "F.Cu") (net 4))
 (segment (start 91.745 35.84) (end 91.745 33.785) (width 0.2) (layer "F.Cu") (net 4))
 (segment (start 88.73375 36.14) (end 91.445 36.14) (width 0.2) (layer "F.Cu") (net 4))
 (segment (start 91.745 33.785) (end 91.3 33.34) (width 0.2) (layer "F.Cu") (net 4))
 (segment (start 86.895 36.265) (end 88.60875 36.265) (width 0.2) (layer "F.Cu") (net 4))
 (segment (start 96.841484 50.7975) (end 99.65 50.7975) (width 1) (layer "F.Cu") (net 1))
 (segment (start 93.271992 47.228008) (end 91.67 48.83) (width 1) (layer "F.Cu") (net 1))
 (segment (start 93.271992 47.228008) (end 96.841484 50.7975) (width 1) (layer "F.Cu") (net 1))
 (segment (start 91.67 48.83) (end 82.03 48.83) (width 1) (layer "F.Cu") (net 1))
 (segment (start 100.12 32.53) (end 100.12 34.24) (width 1) (layer "F.Cu") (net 2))
 (segment (start 97.13 43.37) (end 94.368008 46.131992) (width 1) (layer "F.Cu") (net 2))
 (segment (start 100.12 34.24) (end 97.13 37.23) (width 1) (layer "F.Cu") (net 2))
 (segment (start 97.13 37.23) (end 97.13 43.37) (width 1) (layer "F.Cu") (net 2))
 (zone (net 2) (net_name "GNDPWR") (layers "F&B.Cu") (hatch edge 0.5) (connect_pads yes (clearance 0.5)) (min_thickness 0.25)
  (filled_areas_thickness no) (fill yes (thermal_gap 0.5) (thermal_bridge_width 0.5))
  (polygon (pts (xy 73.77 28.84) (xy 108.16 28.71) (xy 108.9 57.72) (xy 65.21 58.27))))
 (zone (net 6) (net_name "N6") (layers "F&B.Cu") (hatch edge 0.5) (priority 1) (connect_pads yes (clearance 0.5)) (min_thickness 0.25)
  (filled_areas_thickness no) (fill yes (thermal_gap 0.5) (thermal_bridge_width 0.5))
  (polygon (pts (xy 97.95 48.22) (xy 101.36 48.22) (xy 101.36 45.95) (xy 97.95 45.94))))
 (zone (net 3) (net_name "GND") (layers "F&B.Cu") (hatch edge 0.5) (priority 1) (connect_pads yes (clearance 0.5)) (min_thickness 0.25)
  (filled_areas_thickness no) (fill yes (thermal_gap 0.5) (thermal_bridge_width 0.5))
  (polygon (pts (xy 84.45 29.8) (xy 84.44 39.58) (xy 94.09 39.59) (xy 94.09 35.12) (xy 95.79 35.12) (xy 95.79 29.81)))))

